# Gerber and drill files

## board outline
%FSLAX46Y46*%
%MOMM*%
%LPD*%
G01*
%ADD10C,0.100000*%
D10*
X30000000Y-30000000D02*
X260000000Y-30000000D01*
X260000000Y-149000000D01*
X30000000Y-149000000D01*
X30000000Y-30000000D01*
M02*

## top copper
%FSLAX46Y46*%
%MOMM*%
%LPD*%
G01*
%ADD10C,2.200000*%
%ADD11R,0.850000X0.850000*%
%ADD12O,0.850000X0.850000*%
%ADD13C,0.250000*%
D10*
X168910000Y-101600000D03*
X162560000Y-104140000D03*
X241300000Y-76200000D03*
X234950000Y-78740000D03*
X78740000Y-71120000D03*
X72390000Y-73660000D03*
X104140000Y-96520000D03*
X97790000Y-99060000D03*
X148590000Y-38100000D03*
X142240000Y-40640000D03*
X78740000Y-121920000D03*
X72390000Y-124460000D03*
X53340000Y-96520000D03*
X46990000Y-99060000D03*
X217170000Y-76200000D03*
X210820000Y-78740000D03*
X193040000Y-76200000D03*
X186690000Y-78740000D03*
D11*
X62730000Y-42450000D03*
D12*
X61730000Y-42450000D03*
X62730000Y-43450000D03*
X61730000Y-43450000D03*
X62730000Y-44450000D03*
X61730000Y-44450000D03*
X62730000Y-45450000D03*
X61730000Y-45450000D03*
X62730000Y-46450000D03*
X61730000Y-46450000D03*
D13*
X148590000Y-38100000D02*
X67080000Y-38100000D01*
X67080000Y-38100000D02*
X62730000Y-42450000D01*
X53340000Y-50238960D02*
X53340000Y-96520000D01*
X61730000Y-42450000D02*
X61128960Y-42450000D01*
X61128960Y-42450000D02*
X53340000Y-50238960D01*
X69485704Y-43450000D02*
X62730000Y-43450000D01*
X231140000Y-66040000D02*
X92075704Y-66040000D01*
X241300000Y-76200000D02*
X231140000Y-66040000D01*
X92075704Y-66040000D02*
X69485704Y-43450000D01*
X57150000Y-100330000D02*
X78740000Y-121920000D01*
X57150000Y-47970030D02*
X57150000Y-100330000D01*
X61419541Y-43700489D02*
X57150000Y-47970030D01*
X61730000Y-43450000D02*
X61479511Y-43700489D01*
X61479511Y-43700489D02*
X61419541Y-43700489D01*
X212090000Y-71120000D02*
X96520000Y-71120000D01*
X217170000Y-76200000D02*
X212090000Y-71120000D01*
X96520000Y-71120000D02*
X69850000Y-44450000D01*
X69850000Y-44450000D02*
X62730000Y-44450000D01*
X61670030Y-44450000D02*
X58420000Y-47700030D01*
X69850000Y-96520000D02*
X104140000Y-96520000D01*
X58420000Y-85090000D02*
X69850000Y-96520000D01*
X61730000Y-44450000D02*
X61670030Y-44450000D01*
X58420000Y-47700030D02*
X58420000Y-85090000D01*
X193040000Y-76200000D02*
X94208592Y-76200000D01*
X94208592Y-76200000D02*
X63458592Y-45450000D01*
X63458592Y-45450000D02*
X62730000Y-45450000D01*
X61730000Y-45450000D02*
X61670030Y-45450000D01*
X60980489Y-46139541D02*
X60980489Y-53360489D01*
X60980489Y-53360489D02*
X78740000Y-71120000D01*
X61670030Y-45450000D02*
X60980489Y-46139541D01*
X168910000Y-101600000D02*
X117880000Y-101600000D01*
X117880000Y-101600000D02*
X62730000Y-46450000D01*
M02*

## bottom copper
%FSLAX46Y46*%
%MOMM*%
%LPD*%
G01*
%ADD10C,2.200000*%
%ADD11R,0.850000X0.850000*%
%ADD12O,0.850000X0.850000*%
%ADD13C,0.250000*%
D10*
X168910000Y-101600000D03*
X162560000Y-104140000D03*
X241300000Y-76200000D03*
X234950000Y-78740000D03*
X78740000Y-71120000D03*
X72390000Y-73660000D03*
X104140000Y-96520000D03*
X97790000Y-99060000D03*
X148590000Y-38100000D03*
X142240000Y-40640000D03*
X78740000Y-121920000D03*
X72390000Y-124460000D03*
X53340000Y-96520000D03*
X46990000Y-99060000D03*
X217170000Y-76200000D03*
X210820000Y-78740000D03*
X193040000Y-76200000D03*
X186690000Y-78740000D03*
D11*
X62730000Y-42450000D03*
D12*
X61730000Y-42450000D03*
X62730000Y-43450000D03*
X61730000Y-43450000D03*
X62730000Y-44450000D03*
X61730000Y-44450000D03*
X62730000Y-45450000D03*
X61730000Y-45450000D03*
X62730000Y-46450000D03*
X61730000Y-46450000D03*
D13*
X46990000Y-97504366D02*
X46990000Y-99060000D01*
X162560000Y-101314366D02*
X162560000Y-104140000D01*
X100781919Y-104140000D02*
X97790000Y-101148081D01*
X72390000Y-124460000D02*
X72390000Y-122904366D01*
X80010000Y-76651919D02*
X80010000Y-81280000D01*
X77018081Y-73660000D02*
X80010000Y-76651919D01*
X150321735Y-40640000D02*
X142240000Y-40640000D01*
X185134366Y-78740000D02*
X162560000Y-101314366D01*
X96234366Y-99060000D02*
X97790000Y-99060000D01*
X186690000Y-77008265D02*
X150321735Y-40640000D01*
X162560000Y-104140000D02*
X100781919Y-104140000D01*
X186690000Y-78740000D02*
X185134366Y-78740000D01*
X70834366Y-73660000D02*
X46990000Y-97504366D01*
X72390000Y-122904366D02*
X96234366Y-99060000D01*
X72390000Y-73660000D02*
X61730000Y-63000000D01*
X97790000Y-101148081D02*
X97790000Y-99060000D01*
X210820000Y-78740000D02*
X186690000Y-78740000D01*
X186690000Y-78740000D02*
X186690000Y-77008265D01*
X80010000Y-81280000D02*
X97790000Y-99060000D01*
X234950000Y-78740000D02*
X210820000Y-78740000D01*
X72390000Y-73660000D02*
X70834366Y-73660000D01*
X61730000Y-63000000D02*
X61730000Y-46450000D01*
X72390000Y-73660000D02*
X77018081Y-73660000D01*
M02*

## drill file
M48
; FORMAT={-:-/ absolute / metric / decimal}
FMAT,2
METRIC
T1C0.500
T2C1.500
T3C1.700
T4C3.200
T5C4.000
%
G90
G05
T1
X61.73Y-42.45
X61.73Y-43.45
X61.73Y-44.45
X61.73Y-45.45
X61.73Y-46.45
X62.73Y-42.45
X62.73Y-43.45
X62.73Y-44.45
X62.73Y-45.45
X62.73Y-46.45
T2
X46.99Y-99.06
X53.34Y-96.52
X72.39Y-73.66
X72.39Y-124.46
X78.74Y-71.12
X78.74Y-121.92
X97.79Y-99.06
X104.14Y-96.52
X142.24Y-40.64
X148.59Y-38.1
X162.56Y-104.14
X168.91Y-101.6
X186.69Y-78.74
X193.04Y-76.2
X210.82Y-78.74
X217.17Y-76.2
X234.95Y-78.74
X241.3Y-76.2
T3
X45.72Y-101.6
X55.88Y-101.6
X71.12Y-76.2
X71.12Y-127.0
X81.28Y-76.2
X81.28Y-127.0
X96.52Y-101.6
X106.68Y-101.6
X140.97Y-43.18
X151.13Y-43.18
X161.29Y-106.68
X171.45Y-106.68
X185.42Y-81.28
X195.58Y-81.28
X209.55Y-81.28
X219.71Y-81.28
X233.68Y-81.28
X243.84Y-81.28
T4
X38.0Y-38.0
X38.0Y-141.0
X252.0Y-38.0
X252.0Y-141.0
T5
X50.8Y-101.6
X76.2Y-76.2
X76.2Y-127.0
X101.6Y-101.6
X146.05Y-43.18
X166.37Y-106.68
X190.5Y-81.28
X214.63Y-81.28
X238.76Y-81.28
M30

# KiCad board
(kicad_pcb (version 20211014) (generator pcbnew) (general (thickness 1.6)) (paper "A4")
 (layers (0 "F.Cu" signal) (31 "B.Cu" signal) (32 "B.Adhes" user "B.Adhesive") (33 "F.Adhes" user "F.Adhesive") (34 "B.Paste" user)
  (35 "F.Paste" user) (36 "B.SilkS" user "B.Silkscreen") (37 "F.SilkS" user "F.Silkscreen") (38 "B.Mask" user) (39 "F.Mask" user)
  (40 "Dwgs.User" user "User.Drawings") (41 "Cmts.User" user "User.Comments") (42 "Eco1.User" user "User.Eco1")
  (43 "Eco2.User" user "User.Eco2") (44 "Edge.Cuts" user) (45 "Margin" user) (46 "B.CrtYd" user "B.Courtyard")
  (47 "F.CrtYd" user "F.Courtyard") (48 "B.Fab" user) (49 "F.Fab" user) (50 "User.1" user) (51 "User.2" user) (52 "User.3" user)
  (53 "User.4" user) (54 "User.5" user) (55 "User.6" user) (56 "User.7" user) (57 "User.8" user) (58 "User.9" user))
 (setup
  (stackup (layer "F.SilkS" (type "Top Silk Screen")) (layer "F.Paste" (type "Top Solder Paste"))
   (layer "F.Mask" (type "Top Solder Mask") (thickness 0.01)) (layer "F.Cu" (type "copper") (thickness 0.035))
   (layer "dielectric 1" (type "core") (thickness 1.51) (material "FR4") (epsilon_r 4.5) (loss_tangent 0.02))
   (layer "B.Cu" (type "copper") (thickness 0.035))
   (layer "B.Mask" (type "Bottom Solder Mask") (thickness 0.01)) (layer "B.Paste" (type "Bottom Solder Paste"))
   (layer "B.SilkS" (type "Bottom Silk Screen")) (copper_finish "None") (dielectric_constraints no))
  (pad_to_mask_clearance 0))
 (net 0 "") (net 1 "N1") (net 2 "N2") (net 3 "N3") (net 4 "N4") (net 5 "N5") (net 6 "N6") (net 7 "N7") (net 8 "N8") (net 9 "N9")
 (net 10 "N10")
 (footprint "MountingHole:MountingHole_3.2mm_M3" (layer "F.Cu") (at 252 38)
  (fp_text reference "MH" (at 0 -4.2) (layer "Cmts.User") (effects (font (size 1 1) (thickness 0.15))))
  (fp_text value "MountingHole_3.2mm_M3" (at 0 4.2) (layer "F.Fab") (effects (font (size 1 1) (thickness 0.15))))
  (pad "" np_thru_hole circle (at 0 0) (size 3.2 3.2) (drill 3.2) (layers *.Cu *.Mask)))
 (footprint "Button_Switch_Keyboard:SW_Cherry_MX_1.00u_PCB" (layer "F.Cu") (at 168.91 101.6)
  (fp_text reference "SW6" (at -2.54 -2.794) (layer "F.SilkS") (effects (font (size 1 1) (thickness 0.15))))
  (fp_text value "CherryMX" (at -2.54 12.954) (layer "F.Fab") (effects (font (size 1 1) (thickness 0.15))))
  (pad "" np_thru_hole circle (at -7.62 5.08) (size 1.7 1.7) (drill 1.7) (layers *.Cu *.Mask))
  (pad "" np_thru_hole circle (at 2.54 5.08) (size 1.7 1.7) (drill 1.7) (layers *.Cu *.Mask))
  (pad "" np_thru_hole circle (at -2.54 5.08) (size 4 4) (drill 4) (layers *.Cu *.Mask))
  (pad "1" thru_hole circle (at 0 0) (size 2.2 2.2) (drill 1.5) (layers *.Cu *.Mask) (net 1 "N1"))
  (pad "2" thru_hole circle (at -6.35 2.54) (size 2.2 2.2) (drill 1.5) (layers *.Cu *.Mask) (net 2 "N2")))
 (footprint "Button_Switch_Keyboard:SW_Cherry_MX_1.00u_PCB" (layer "F.Cu") (at 241.3 76.2)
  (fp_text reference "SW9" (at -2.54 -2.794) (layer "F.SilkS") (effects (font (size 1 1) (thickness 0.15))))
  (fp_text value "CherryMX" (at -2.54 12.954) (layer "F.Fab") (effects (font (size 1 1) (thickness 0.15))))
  (pad "" np_thru_hole circle (at -7.62 5.08) (size 1.7 1.7) (drill 1.7) (layers *.Cu *.Mask))
  (pad "" np_thru_hole circle (at 2.54 5.08) (size 1.7 1.7) (drill 1.7) (layers *.Cu *.Mask))
  (pad "" np_thru_hole circle (at -2.54 5.08) (size 4 4) (drill 4) (layers *.Cu *.Mask))
  (pad "1" thru_hole circle (at 0 0) (size 2.2 2.2) (drill 1.5) (layers *.Cu *.Mask) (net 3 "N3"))
  (pad "2" thru_hole circle (at -6.35 2.54) (size 2.2 2.2) (drill 1.5) (layers *.Cu *.Mask) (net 2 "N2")))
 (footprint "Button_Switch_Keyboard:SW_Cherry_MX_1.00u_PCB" (layer "F.Cu") (at 78.74 71.12)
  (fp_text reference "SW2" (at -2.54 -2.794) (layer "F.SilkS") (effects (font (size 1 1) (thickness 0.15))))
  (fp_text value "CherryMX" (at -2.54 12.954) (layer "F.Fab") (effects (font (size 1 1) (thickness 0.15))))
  (pad "" np_thru_hole circle (at 2.54 5.08) (size 1.7 1.7) (drill 1.7) (layers *.Cu *.Mask))
  (pad "" np_thru_hole circle (at -2.54 5.08) (size 4 4) (drill 4) (layers *.Cu *.Mask))
  (pad "" np_thru_hole circle (at -7.62 5.08) (size 1.7 1.7) (drill 1.7) (layers *.Cu *.Mask))
  (pad "1" thru_hole circle (at 0 0) (size 2.2 2.2) (drill 1.5) (layers *.Cu *.Mask) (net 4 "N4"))
  (pad "2" thru_hole circle (at -6.35 2.54) (size 2.2 2.2) (drill 1.5) (layers *.Cu *.Mask) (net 2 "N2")))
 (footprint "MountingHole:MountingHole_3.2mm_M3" (layer "F.Cu") (at 252 141)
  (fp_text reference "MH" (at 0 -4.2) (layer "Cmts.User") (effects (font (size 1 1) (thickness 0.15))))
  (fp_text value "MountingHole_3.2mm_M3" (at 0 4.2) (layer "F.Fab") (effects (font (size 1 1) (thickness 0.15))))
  (pad "" np_thru_hole circle (at 0 0) (size 3.2 3.2) (drill 3.2) (layers *.Cu *.Mask)))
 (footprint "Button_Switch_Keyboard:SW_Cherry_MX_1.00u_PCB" (layer "F.Cu") (at 104.14 96.52)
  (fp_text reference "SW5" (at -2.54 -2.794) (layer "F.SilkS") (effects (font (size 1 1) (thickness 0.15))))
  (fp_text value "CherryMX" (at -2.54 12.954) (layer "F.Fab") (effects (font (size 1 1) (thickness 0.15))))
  (pad "" np_thru_hole circle (at 2.54 5.08) (size 1.7 1.7) (drill 1.7) (layers *.Cu *.Mask))
  (pad "" np_thru_hole circle (at -7.62 5.08) (size 1.7 1.7) (drill 1.7) (layers *.Cu *.Mask))
  (pad "" np_thru_hole circle (at -2.54 5.08) (size 4 4) (drill 4) (layers *.Cu *.Mask))
  (pad "1" thru_hole circle (at 0 0) (size 2.2 2.2) (drill 1.5) (layers *.Cu *.Mask) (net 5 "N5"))
  (pad "2" thru_hole circle (at -6.35 2.54) (size 2.2 2.2) (drill 1.5) (layers *.Cu *.Mask) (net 2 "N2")))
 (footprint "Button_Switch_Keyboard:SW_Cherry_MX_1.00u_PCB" (layer "F.Cu") (at 148.59 38.1)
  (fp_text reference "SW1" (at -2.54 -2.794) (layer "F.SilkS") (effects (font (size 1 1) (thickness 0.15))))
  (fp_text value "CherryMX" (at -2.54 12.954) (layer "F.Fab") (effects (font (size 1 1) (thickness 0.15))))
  (pad "" np_thru_hole circle (at -2.54 5.08) (size 4 4) (drill 4) (layers *.Cu *.Mask))
  (pad "" np_thru_hole circle (at -7.62 5.08) (size 1.7 1.7) (drill 1.7) (layers *.Cu *.Mask))
  (pad "" np_thru_hole circle (at 2.54 5.08) (size 1.7 1.7) (drill 1.7) (layers *.Cu *.Mask))
  (pad "1" thru_hole circle (at 0 0) (size 2.2 2.2) (drill 1.5) (layers *.Cu *.Mask) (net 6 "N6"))
  (pad "2" thru_hole circle (at -6.35 2.54) (size 2.2 2.2) (drill 1.5) (layers *.Cu *.Mask) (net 2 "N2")))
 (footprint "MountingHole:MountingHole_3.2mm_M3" (layer "F.Cu") (at 38 38)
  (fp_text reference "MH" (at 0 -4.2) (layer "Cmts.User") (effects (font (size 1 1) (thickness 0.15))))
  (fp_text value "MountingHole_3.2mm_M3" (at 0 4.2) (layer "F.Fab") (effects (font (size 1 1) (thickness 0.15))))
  (pad "" np_thru_hole circle (at 0 0) (size 3.2 3.2) (drill 3.2) (layers *.Cu *.Mask)))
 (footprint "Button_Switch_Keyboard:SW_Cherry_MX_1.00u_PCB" (layer "F.Cu") (at 78.74 121.92)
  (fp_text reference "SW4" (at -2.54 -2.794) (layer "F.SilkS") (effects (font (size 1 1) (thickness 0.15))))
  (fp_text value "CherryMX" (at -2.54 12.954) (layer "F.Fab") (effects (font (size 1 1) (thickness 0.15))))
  (pad "" np_thru_hole circle (at -7.62 5.08) (size 1.7 1.7) (drill 1.7) (layers *.Cu *.Mask))
  (pad "" np_thru_hole circle (at -2.54 5.08) (size 4 4) (drill 4) (layers *.Cu *.Mask))
  (pad "" np_thru_hole circle (at 2.54 5.08) (size 1.7 1.7) (drill 1.7) (layers *.Cu *.Mask))
  (pad "1" thru_hole circle (at 0 0) (size 2.2 2.2) (drill 1.5) (layers *.Cu *.Mask) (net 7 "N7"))
  (pad "2" thru_hole circle (at -6.35 2.54) (size 2.2 2.2) (drill 1.5) (layers *.Cu *.Mask) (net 2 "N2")))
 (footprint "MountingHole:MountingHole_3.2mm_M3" (layer "F.Cu") (at 38 141)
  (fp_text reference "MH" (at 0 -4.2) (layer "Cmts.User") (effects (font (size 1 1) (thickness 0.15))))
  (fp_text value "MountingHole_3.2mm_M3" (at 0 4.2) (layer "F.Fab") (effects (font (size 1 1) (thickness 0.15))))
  (pad "" np_thru_hole circle (at 0 0) (size 3.2 3.2) (drill 3.2) (layers *.Cu *.Mask)))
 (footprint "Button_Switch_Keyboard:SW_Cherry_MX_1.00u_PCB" (layer "F.Cu") (at 53.34 96.52)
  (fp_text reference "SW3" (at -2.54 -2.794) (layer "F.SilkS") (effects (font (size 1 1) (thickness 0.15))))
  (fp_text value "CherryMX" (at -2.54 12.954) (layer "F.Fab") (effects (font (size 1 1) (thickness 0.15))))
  (pad "" np_thru_hole circle (at 2.54 5.08) (size 1.7 1.7) (drill 1.7) (layers *.Cu *.Mask))
  (pad "" np_thru_hole circle (at -2.54 5.08) (size 4 4) (drill 4) (layers *.Cu *.Mask))
  (pad "" np_thru_hole circle (at -7.62 5.08) (size 1.7 1.7) (drill 1.7) (layers *.Cu *.Mask))
  (pad "1" thru_hole circle (at 0 0) (size 2.2 2.2) (drill 1.5) (layers *.Cu *.Mask) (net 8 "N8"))
  (pad "2" thru_hole circle (at -6.35 2.54) (size 2.2 2.2) (drill 1.5) (layers *.Cu *.Mask) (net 2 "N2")))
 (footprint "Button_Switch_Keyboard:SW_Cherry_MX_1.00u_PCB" (layer "F.Cu") (at 217.17 76.2)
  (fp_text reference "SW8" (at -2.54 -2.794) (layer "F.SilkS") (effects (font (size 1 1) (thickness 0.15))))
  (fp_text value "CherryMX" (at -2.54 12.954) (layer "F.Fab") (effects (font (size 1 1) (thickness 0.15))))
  (pad "" np_thru_hole circle (at -2.54 5.08) (size 4 4) (drill 4) (layers *.Cu *.Mask))
  (pad "" np_thru_hole circle (at -7.62 5.08) (size 1.7 1.7) (drill 1.7) (layers *.Cu *.Mask))
  (pad "" np_thru_hole circle (at 2.54 5.08) (size 1.7 1.7) (drill 1.7) (layers *.Cu *.Mask))
  (pad "1" thru_hole circle (at 0 0) (size 2.2 2.2) (drill 1.5) (layers *.Cu *.Mask) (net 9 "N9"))
  (pad "2" thru_hole circle (at -6.35 2.54) (size 2.2 2.2) (drill 1.5) (layers *.Cu *.Mask) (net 2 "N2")))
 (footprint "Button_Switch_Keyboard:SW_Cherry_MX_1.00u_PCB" (layer "F.Cu") (at 193.04 76.2)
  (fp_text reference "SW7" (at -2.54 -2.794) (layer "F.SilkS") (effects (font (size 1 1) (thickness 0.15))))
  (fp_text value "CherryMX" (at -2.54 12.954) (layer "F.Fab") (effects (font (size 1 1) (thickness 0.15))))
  (pad "" np_thru_hole circle (at 2.54 5.08) (size 1.7 1.7) (drill 1.7) (layers *.Cu *.Mask))
  (pad "" np_thru_hole circle (at -7.62 5.08) (size 1.7 1.7) (drill 1.7) (layers *.Cu *.Mask))
  (pad "" np_thru_hole circle (at -2.54 5.08) (size 4 4) (drill 4) (layers *.Cu *.Mask))
  (pad "1" thru_hole circle (at 0 0) (size 2.2 2.2) (drill 1.5) (layers *.Cu *.Mask) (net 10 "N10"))
  (pad "2" thru_hole circle (at -6.35 2.54) (size 2.2 2.2) (drill 1.5) (layers *.Cu *.Mask) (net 2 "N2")))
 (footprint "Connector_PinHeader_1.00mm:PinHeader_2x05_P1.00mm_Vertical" (layer "B.Cu") (at 62.73 42.45 180)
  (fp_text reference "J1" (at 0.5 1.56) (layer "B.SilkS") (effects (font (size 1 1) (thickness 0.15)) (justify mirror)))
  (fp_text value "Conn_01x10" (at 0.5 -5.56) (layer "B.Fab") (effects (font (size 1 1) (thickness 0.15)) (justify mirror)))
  (pad "1" thru_hole rect (at 0 0 180) (size 0.85 0.85) (drill 0.5) (layers *.Cu *.Mask) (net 6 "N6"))
  (pad "2" thru_hole oval (at 1 0 180) (size 0.85 0.85) (drill 0.5) (layers *.Cu *.Mask) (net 8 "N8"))
  (pad "3" thru_hole oval (at 0 -1 180) (size 0.85 0.85) (drill 0.5) (layers *.Cu *.Mask) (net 3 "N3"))
  (pad "4" thru_hole oval (at 1 -1 180) (size 0.85 0.85) (drill 0.5) (layers *.Cu *.Mask) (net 7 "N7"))
  (pad "5" thru_hole oval (at 0 -2 180) (size 0.85 0.85) (drill 0.5) (layers *.Cu *.Mask) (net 9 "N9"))
  (pad "6" thru_hole oval (at 1 -2 180) (size 0.85 0.85) (drill 0.5) (layers *.Cu *.Mask) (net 5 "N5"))
  (pad "7" thru_hole oval (at 0 -3 180) (size 0.85 0.85) (drill 0.5) (layers *.Cu *.Mask) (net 10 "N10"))
  (pad "8" thru_hole oval (at 1 -3 180) (size 0.85 0.85) (drill 0.5) (layers *.Cu *.Mask) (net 4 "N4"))
  (pad "9" thru_hole oval (at 0 -4 180) (size 0.85 0.85) (drill 0.5) (layers *.Cu *.Mask) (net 1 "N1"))
  (pad "10" thru_hole oval (at 1 -4 180) (size 0.85 0.85) (drill 0.5) (layers *.Cu *.Mask) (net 2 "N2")))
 (gr_rect (start 30 149) (end 260 30) (layer "Edge.Cuts") (width 0.1) (fill none))
 (segment (start 148.59 38.1) (end 67.08 38.1) (width 0.25) (layer "F.Cu") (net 6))
 (segment (start 67.08 38.1) (end 62.73 42.45) (width 0.25) (layer "F.Cu") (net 6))
 (segment (start 53.34 50.23896) (end 53.34 96.52) (width 0.25) (layer "F.Cu") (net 8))
 (segment (start 61.73 42.45) (end 61.12896 42.45) (width 0.25) (layer "F.Cu") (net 8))
 (segment (start 61.12896 42.45) (end 53.34 50.23896) (width 0.25) (layer "F.Cu") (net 8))
 (segment (start 69.485704 43.45) (end 62.73 43.45) (width 0.25) (layer "F.Cu") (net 3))
 (segment (start 231.14 66.04) (end 92.075704 66.04) (width 0.25) (layer "F.Cu") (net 3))
 (segment (start 241.3 76.2) (end 231.14 66.04) (width 0.25) (layer "F.Cu") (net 3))
 (segment (start 92.075704 66.04) (end 69.485704 43.45) (width 0.25) (layer "F.Cu") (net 3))
 (segment (start 57.15 100.33) (end 78.74 121.92) (width 0.25) (layer "F.Cu") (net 7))
 (segment (start 57.15 47.97003) (end 57.15 100.33) (width 0.25) (layer "F.Cu") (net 7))
 (segment (start 61.419541 43.700489) (end 57.15 47.97003) (width 0.25) (layer "F.Cu") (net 7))
 (segment (start 61.73 43.45) (end 61.479511 43.700489) (width 0.25) (layer "F.Cu") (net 7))
 (segment (start 61.479511 43.700489) (end 61.419541 43.700489) (width 0.25) (layer "F.Cu") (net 7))
 (segment (start 212.09 71.12) (end 96.52 71.12) (width 0.25) (layer "F.Cu") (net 9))
 (segment (start 217.17 76.2) (end 212.09 71.12) (width 0.25) (layer "F.Cu") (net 9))
 (segment (start 96.52 71.12) (end 69.85 44.45) (width 0.25) (layer "F.Cu") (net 9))
 (segment (start 69.85 44.45) (end 62.73 44.45) (width 0.25) (layer "F.Cu") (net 9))
 (segment (start 61.67003 44.45) (end 58.42 47.70003) (width 0.25) (layer "F.Cu") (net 5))
 (segment (start 69.85 96.52) (end 104.14 96.52) (width 0.25) (layer "F.Cu") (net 5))
 (segment (start 58.42 85.09) (end 69.85 96.52) (width 0.25) (layer "F.Cu") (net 5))
 (segment (start 61.73 44.45) (end 61.67003 44.45) (width 0.25) (layer "F.Cu") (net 5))
 (segment (start 58.42 47.70003) (end 58.42 85.09) (width 0.25) (layer "F.Cu") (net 5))
 (segment (start 193.04 76.2) (end 94.208592 76.2) (width 0.25) (layer "F.Cu") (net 10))
 (segment (start 94.208592 76.2) (end 63.458592 45.45) (width 0.25) (layer "F.Cu") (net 10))
 (segment (start 63.458592 45.45) (end 62.73 45.45) (width 0.25) (layer "F.Cu") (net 10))
 (segment (start 61.73 45.45) (end 61.67003 45.45) (width 0.25) (layer "F.Cu") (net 4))
 (segment (start 60.980489 46.139541) (end 60.980489 53.360489) (width 0.25) (layer "F.Cu") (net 4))
 (segment (start 60.980489 53.360489) (end 78.74 71.12) (width 0.25) (layer "F.Cu") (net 4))
 (segment (start 61.67003 45.45) (end 60.980489 46.139541) (width 0.25) (layer "F.Cu") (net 4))
 (segment (start 168.91 101.6) (end 117.88 101.6) (width 0.25) (layer "F.Cu") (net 1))
 (segment (start 117.88 101.6) (end 62.73 46.45) (width 0.25) (layer "F.Cu") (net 1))
 (segment (start 46.99 97.504366) (end 46.99 99.06) (width 0.25) (layer "B.Cu") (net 2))
 (segment (start 162.56 101.314366) (end 162.56 104.14) (width 0.25) (layer "B.Cu") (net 2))
 (segment (start 100.781919 104.14) (end 97.79 101.148081) (width 0.25) (layer "B.Cu") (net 2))
 (segment (start 72.39 124.46) (end 72.39 122.904366) (width 0.25) (layer "B.Cu") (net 2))
 (segment (start 80.01 76.651919) (end 80.01 81.28) (width 0.25) (layer "B.Cu") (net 2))
 (segment (start 77.018081 73.66) (end 80.01 76.651919) (width 0.25) (layer "B.Cu") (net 2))
 (segment (start 150.321735 40.64) (end 142.24 40.64) (width 0.25) (layer "B.Cu") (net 2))
 (segment (start 185.134366 78.74) (end 162.56 101.314366) (width 0.25) (layer "B.Cu") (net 2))
 (segment (start 96.234366 99.06) (end 97.79 99.06) (width 0.25) (layer "B.Cu") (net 2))
 (segment (start 186.69 77.008265) (end 150.321735 40.64) (width 0.25) (layer "B.Cu") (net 2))
 (segment (start 162.56 104.14) (end 100.781919 104.14) (width 0.25) (layer "B.Cu") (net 2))
 (segment (start 186.69 78.74) (end 185.134366 78.74) (width 0.25) (layer "B.Cu") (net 2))
 (segment (start 70.834366 73.66) (end 46.99 97.504366) (width 0.25) (layer "B.Cu") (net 2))
 (segment (start 72.39 122.904366) (end 96.234366 99.06) (width 0.25) (layer "B.Cu") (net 2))
 (segment (start 72.39 73.66) (end 61.73 63) (width 0.25) (layer "B.Cu") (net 2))
 (segment (start 97.79 101.148081) (end 97.79 99.06) (width 0.25) (layer "B.Cu") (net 2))
 (segment (start 210.82 78.74) (end 186.69 78.74) (width 0.25) (layer "B.Cu") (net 2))
 (segment (start 186.69 78.74) (end 186.69 77.008265) (width 0.25) (layer "B.Cu") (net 2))
 (segment (start 80.01 81.28) (end 97.79 99.06) (width 0.25) (layer "B.Cu") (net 2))
 (segment (start 234.95 78.74) (end 210.82 78.74) (width 0.25) (layer "B.Cu") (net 2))
 (segment (start 72.39 73.66) (end 70.834366 73.66) (width 0.25) (layer "B.Cu") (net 2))
 (segment (start 61.73 63) (end 61.73 46.45) (width 0.25) (layer "B.Cu") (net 2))
 (segment (start 72.39 73.66) (end 77.018081 73.66) (width 0.25) (layer "B.Cu") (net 2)))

